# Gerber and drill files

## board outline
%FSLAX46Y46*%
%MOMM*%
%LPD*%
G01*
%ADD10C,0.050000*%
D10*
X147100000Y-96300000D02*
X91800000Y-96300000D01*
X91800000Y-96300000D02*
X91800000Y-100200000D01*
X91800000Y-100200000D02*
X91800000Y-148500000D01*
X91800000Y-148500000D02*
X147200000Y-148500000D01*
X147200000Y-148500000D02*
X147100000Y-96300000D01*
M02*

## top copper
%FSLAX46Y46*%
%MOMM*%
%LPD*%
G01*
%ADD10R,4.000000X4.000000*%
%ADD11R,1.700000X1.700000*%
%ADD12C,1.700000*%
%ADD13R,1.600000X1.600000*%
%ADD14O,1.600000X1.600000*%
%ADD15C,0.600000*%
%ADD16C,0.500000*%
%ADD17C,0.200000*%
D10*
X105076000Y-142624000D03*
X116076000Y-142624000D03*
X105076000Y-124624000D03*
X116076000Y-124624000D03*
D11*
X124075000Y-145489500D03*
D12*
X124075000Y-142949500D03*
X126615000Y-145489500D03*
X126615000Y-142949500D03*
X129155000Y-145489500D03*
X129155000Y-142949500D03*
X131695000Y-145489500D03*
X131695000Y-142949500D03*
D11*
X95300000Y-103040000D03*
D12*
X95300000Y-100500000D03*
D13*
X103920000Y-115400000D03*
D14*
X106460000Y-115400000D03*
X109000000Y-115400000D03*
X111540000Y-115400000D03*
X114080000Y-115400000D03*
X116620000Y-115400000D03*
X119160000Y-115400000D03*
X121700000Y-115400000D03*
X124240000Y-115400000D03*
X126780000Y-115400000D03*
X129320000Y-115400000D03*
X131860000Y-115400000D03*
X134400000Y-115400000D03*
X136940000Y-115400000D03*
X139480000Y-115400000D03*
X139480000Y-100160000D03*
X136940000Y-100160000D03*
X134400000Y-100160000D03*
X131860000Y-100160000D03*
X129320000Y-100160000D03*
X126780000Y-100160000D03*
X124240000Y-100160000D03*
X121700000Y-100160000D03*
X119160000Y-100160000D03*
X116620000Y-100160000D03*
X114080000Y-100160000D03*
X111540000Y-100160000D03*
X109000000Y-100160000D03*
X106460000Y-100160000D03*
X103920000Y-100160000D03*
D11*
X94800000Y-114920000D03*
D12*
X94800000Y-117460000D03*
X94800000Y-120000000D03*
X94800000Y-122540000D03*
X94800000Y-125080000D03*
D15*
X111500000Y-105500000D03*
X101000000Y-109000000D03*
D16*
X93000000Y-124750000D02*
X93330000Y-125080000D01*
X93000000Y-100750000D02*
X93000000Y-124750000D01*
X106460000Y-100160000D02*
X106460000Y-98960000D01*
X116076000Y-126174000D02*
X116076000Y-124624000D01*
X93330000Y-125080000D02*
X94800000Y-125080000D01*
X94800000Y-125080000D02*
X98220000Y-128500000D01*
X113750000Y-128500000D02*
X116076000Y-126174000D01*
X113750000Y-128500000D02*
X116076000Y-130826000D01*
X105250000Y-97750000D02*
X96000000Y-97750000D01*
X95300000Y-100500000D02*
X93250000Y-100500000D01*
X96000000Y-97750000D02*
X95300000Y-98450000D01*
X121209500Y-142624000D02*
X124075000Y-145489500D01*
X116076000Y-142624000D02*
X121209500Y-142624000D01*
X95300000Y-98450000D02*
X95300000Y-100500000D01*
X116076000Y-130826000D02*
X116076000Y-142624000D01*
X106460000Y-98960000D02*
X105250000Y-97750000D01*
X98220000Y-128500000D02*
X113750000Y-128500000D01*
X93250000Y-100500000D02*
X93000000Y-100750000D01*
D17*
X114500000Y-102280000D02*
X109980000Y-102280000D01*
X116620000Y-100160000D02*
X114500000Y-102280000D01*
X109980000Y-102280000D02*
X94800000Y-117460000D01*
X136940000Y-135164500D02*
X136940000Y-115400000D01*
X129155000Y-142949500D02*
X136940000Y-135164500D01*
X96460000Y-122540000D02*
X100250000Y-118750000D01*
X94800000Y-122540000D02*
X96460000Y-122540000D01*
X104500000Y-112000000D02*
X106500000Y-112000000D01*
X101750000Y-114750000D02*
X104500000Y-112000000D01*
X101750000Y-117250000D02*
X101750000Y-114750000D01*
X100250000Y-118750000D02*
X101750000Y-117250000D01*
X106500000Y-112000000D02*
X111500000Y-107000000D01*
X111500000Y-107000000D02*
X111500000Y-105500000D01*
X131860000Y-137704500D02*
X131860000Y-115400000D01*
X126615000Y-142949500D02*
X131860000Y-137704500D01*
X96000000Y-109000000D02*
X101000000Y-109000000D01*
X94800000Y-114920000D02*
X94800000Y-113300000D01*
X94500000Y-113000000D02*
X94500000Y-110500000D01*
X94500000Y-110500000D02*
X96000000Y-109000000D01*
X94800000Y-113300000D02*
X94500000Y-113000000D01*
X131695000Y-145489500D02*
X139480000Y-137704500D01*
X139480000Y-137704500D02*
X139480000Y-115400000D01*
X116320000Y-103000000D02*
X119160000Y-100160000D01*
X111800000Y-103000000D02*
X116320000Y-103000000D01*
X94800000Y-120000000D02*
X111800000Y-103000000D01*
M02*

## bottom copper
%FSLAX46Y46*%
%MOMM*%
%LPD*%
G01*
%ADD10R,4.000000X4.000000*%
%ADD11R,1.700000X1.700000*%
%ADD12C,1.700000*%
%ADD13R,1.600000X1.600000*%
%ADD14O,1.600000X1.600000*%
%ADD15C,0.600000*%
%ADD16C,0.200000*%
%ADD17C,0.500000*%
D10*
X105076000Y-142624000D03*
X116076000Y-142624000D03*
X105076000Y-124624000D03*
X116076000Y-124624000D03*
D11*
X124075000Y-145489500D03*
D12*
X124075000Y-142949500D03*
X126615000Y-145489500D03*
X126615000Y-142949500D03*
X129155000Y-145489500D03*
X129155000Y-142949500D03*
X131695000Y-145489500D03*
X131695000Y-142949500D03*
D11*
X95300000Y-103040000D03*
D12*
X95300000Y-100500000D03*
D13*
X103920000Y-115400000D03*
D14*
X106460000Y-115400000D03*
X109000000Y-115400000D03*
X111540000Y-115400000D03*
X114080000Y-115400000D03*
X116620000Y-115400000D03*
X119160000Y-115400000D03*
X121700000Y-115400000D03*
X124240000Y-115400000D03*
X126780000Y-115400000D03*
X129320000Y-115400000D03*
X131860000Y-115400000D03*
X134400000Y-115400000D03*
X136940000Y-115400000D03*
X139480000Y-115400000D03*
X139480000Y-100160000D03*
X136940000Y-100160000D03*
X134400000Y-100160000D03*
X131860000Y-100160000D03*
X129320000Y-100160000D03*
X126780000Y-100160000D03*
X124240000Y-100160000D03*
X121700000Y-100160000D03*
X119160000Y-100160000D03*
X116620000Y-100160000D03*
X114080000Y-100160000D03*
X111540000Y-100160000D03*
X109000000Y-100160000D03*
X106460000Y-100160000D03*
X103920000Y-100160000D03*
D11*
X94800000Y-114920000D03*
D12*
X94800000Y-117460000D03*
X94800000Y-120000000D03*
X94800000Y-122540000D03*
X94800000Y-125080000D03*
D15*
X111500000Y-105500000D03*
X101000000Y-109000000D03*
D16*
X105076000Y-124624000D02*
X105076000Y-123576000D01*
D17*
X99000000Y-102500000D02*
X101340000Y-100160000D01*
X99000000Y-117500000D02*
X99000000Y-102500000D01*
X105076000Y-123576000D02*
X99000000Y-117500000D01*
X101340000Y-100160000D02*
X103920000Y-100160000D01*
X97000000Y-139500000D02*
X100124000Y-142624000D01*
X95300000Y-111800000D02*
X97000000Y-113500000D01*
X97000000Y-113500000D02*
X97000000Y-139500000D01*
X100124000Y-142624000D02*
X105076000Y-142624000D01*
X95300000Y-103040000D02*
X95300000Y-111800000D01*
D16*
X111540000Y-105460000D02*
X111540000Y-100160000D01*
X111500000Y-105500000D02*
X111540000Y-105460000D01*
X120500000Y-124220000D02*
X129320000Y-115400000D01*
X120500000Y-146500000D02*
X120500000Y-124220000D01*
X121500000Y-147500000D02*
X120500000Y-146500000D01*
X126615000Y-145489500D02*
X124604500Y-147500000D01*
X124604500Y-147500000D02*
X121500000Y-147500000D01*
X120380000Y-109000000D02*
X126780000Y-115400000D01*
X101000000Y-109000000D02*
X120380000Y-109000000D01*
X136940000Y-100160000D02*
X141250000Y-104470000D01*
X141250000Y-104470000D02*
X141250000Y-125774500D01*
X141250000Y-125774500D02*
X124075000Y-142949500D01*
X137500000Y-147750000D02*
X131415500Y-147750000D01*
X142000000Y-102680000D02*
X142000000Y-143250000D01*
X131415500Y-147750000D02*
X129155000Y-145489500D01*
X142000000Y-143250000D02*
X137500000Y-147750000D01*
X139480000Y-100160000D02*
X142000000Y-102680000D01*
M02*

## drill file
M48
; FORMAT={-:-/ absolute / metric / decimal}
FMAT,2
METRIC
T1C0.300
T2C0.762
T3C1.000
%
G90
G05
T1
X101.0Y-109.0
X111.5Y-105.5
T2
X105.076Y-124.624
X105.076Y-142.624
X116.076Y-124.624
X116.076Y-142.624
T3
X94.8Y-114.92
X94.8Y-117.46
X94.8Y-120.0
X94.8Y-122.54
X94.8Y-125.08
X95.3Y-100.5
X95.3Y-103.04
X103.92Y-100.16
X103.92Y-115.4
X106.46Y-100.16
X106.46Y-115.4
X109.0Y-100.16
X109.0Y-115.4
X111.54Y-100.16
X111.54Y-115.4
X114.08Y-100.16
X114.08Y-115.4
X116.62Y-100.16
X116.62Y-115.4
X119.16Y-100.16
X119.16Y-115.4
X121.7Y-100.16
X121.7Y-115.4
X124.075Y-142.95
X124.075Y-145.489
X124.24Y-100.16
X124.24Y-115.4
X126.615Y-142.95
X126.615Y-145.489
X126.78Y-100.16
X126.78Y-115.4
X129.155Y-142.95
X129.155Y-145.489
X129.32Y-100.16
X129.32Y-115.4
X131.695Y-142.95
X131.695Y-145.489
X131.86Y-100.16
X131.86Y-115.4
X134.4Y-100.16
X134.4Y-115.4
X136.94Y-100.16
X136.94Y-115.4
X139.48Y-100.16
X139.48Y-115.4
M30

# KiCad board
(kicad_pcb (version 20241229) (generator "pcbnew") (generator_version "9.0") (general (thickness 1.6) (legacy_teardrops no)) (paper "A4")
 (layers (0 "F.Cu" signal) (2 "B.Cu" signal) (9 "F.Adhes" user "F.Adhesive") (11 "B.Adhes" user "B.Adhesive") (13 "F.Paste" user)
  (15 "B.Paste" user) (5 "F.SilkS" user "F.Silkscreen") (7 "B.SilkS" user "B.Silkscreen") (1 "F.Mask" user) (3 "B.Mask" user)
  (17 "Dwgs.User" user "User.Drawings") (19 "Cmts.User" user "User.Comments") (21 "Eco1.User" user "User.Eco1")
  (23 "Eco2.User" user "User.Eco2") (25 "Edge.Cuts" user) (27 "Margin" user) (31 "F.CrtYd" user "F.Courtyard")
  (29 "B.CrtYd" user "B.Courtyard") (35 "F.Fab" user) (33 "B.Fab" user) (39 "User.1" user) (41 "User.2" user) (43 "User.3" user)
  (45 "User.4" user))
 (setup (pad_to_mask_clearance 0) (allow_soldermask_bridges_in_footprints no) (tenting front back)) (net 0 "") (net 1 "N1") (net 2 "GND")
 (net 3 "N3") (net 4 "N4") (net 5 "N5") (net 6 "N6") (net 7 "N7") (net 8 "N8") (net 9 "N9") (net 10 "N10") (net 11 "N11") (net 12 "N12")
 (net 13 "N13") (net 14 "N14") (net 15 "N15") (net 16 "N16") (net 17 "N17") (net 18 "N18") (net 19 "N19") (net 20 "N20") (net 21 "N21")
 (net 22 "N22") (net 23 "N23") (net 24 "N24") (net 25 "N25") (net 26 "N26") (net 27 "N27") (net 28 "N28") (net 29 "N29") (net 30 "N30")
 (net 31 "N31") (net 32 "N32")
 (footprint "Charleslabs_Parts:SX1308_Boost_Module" (layer "F.Cu") (at 105.124 142.576 90)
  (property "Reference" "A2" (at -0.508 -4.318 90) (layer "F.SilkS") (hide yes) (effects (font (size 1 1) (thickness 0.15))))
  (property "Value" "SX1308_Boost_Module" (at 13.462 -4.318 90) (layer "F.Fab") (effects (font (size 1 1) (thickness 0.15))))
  (pad "1" thru_hole rect (at -0.048 -0.048 90) (size 4 4) (drill 0.762) (layers "*.Cu" "*.Mask") (remove_unused_layers no) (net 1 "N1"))
  (pad "2" thru_hole rect (at -0.048 10.952 90) (size 4 4) (drill 0.762) (layers "*.Cu" "*.Mask") (remove_unused_layers no) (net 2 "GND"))
  (pad "3" thru_hole rect (at 17.952 -0.048 90) (size 4 4) (drill 0.762) (layers "*.Cu" "*.Mask") (remove_unused_layers no) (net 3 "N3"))
  (pad "4" thru_hole rect (at 17.952 10.952 90) (size 4 4) (drill 0.762) (layers "*.Cu" "*.Mask") (remove_unused_layers no) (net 2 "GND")))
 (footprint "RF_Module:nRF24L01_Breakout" (layer "F.Cu") (at 124.075 145.4895 90)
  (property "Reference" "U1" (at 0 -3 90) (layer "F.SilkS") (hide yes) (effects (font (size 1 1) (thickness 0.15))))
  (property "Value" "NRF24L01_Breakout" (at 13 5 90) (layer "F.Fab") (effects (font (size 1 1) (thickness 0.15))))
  (pad "1" thru_hole rect (at 0 0 90) (size 1.7 1.7) (drill 1) (layers "*.Cu" "*.Mask") (remove_unused_layers no) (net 2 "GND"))
  (pad "2" thru_hole circle (at 2.54 0 90) (size 1.7 1.7) (drill 1) (layers "*.Cu" "*.Mask") (remove_unused_layers no) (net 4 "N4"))
  (pad "3" thru_hole circle (at 0 2.54 90) (size 1.7 1.7) (drill 1) (layers "*.Cu" "*.Mask") (remove_unused_layers no) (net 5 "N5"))
  (pad "4" thru_hole circle (at 2.54 2.54 90) (size 1.7 1.7) (drill 1) (layers "*.Cu" "*.Mask") (remove_unused_layers no) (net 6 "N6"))
  (pad "5" thru_hole circle (at 0 5.08 90) (size 1.7 1.7) (drill 1) (layers "*.Cu" "*.Mask") (remove_unused_layers no) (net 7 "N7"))
  (pad "6" thru_hole circle (at 2.54 5.08 90) (size 1.7 1.7) (drill 1) (layers "*.Cu" "*.Mask") (remove_unused_layers no) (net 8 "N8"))
  (pad "7" thru_hole circle (at 0 7.62 90) (size 1.7 1.7) (drill 1) (layers "*.Cu" "*.Mask") (remove_unused_layers no) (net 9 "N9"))
  (pad "8" thru_hole circle (at 2.54 7.62 90) (size 1.7 1.7) (drill 1) (layers "*.Cu" "*.Mask") (remove_unused_layers no) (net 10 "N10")))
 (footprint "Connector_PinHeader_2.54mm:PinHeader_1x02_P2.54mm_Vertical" (layer "F.Cu") (at 95.3 103.04 180)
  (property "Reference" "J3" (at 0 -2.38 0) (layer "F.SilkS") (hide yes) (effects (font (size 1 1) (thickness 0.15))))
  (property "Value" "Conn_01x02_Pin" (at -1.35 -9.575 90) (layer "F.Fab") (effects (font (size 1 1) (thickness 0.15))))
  (pad "1" thru_hole rect (at 0 0 180) (size 1.7 1.7) (drill 1) (layers "*.Cu" "*.Mask") (remove_unused_layers no) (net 1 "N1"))
  (pad "2" thru_hole circle (at 0 2.54 180) (size 1.7 1.7) (drill 1) (layers "*.Cu" "*.Mask") (remove_unused_layers no) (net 2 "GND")))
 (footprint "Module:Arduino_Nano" (layer "F.Cu") (at 103.92 115.4 90)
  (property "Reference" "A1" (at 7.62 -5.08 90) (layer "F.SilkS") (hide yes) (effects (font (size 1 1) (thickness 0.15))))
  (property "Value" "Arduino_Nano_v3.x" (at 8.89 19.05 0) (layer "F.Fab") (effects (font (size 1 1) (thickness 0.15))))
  (pad "1" thru_hole rect (at 0 0 90) (size 1.6 1.6) (drill 1) (layers "*.Cu" "*.Mask") (remove_unused_layers no) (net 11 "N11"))
  (pad "2" thru_hole oval (at 0 2.54 90) (size 1.6 1.6) (drill 1) (layers "*.Cu" "*.Mask") (remove_unused_layers no) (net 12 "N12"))
  (pad "3" thru_hole oval (at 0 5.08 90) (size 1.6 1.6) (drill 1) (layers "*.Cu" "*.Mask") (remove_unused_layers no) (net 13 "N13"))
  (pad "4" thru_hole oval (at 0 7.62 90) (size 1.6 1.6) (drill 1) (layers "*.Cu" "*.Mask") (remove_unused_layers no) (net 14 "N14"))
  (pad "5" thru_hole oval (at 0 10.16 90) (size 1.6 1.6) (drill 1) (layers "*.Cu" "*.Mask") (remove_unused_layers no) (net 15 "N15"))
  (pad "6" thru_hole oval (at 0 12.7 90) (size 1.6 1.6) (drill 1) (layers "*.Cu" "*.Mask") (remove_unused_layers no) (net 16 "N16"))
  (pad "7" thru_hole oval (at 0 15.24 90) (size 1.6 1.6) (drill 1) (layers "*.Cu" "*.Mask") (remove_unused_layers no) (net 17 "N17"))
  (pad "8" thru_hole oval (at 0 17.78 90) (size 1.6 1.6) (drill 1) (layers "*.Cu" "*.Mask") (remove_unused_layers no) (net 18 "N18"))
  (pad "9" thru_hole oval (at 0 20.32 90) (size 1.6 1.6) (drill 1) (layers "*.Cu" "*.Mask") (remove_unused_layers no) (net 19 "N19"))
  (pad "10" thru_hole oval (at 0 22.86 90) (size 1.6 1.6) (drill 1) (layers "*.Cu" "*.Mask") (remove_unused_layers no) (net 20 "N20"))
  (pad "11" thru_hole oval (at 0 25.4 90) (size 1.6 1.6) (drill 1) (layers "*.Cu" "*.Mask") (remove_unused_layers no) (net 5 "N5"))
  (pad "12" thru_hole oval (at 0 27.94 90) (size 1.6 1.6) (drill 1) (layers "*.Cu" "*.Mask") (remove_unused_layers no) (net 6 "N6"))
  (pad "13" thru_hole oval (at 0 30.48 90) (size 1.6 1.6) (drill 1) (layers "*.Cu" "*.Mask") (remove_unused_layers no) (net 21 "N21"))
  (pad "14" thru_hole oval (at 0 33.02 90) (size 1.6 1.6) (drill 1) (layers "*.Cu" "*.Mask") (remove_unused_layers no) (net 8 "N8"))
  (pad "15" thru_hole oval (at 0 35.56 90) (size 1.6 1.6) (drill 1) (layers "*.Cu" "*.Mask") (remove_unused_layers no) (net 9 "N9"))
  (pad "16" thru_hole oval (at 15.24 35.56 90) (size 1.6 1.6) (drill 1) (layers "*.Cu" "*.Mask") (remove_unused_layers no) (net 7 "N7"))
  (pad "17" thru_hole oval (at 15.24 33.02 90) (size 1.6 1.6) (drill 1) (layers "*.Cu" "*.Mask") (remove_unused_layers no) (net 4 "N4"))
  (pad "18" thru_hole oval (at 15.24 30.48 90) (size 1.6 1.6) (drill 1) (layers "*.Cu" "*.Mask") (remove_unused_layers no) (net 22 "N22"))
  (pad "19" thru_hole oval (at 15.24 27.94 90) (size 1.6 1.6) (drill 1) (layers "*.Cu" "*.Mask") (remove_unused_layers no) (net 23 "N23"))
  (pad "20" thru_hole oval (at 15.24 25.4 90) (size 1.6 1.6) (drill 1) (layers "*.Cu" "*.Mask") (remove_unused_layers no) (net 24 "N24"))
  (pad "21" thru_hole oval (at 15.24 22.86 90) (size 1.6 1.6) (drill 1) (layers "*.Cu" "*.Mask") (remove_unused_layers no) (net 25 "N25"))
  (pad "22" thru_hole oval (at 15.24 20.32 90) (size 1.6 1.6) (drill 1) (layers "*.Cu" "*.Mask") (remove_unused_layers no) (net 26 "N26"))
  (pad "23" thru_hole oval (at 15.24 17.78 90) (size 1.6 1.6) (drill 1) (layers "*.Cu" "*.Mask") (remove_unused_layers no) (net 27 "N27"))
  (pad "24" thru_hole oval (at 15.24 15.24 90) (size 1.6 1.6) (drill 1) (layers "*.Cu" "*.Mask") (remove_unused_layers no) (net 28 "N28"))
  (pad "25" thru_hole oval (at 15.24 12.7 90) (size 1.6 1.6) (drill 1) (layers "*.Cu" "*.Mask") (remove_unused_layers no) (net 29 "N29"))
  (pad "26" thru_hole oval (at 15.24 10.16 90) (size 1.6 1.6) (drill 1) (layers "*.Cu" "*.Mask") (remove_unused_layers no) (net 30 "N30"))
  (pad "27" thru_hole oval (at 15.24 7.62 90) (size 1.6 1.6) (drill 1) (layers "*.Cu" "*.Mask") (remove_unused_layers no) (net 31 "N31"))
  (pad "28" thru_hole oval (at 15.24 5.08 90) (size 1.6 1.6) (drill 1) (layers "*.Cu" "*.Mask") (remove_unused_layers no) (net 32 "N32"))
  (pad "29" thru_hole oval (at 15.24 2.54 90) (size 1.6 1.6) (drill 1) (layers "*.Cu" "*.Mask") (remove_unused_layers no) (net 2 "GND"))
  (pad "30" thru_hole oval (at 15.24 0 90) (size 1.6 1.6) (drill 1) (layers "*.Cu" "*.Mask") (remove_unused_layers no) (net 3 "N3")))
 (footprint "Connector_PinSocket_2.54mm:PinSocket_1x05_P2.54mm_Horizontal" (layer "F.Cu") (at 94.8 114.92)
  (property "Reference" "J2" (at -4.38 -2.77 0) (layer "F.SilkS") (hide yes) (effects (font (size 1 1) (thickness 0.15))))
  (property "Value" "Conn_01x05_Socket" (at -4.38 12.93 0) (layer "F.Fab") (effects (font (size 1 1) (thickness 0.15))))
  (pad "1" thru_hole rect (at 0 0) (size 1.7 1.7) (drill 1) (layers "*.Cu" "*.Mask") (remove_unused_layers no) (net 20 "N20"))
  (pad "2" thru_hole circle (at 0 2.54) (size 1.7 1.7) (drill 1) (layers "*.Cu" "*.Mask") (remove_unused_layers no) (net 29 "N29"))
  (pad "3" thru_hole circle (at 0 5.08) (size 1.7 1.7) (drill 1) (layers "*.Cu" "*.Mask") (remove_unused_layers no) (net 28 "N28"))
  (pad "4" thru_hole circle (at 0 7.62) (size 1.7 1.7) (drill 1) (layers "*.Cu" "*.Mask") (remove_unused_layers no) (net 31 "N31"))
  (pad "5" thru_hole circle (at 0 10.16) (size 1.7 1.7) (drill 1) (layers "*.Cu" "*.Mask") (remove_unused_layers no) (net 2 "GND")))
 (gr_line (start 147.1 96.3) (end 91.8 96.3) (stroke (width 0.05) (type default)) (layer "Edge.Cuts"))
 (gr_line (start 91.8 96.3) (end 91.8 100.2) (stroke (width 0.05) (type default)) (layer "Edge.Cuts"))
 (gr_line (start 91.8 100.2) (end 91.8 148.5) (stroke (width 0.05) (type default)) (layer "Edge.Cuts"))
 (gr_line (start 91.8 148.5) (end 147.2 148.5) (stroke (width 0.05) (type default)) (layer "Edge.Cuts"))
 (gr_line (start 147.2 148.5) (end 147.1 96.3) (stroke (width 0.05) (type default)) (layer "Edge.Cuts"))
 (segment (start 93 124.75) (end 93.33 125.08) (width 0.5) (layer "F.Cu") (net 2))
 (segment (start 93 100.75) (end 93 124.75) (width 0.5) (layer "F.Cu") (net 2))
 (segment (start 106.46 100.16) (end 106.46 98.96) (width 0.5) (layer "F.Cu") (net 2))
 (segment (start 116.076 126.174) (end 116.076 124.624) (width 0.5) (layer "F.Cu") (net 2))
 (segment (start 93.33 125.08) (end 94.8 125.08) (width 0.5) (layer "F.Cu") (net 2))
 (segment (start 94.8 125.08) (end 98.22 128.5) (width 0.5) (layer "F.Cu") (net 2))
 (segment (start 113.75 128.5) (end 116.076 126.174) (width 0.5) (layer "F.Cu") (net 2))
 (segment (start 113.75 128.5) (end 116.076 130.826) (width 0.5) (layer "F.Cu") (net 2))
 (segment (start 105.25 97.75) (end 96 97.75) (width 0.5) (layer "F.Cu") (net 2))
 (segment (start 95.3 100.5) (end 93.25 100.5) (width 0.5) (layer "F.Cu") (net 2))
 (segment (start 96 97.75) (end 95.3 98.45) (width 0.5) (layer "F.Cu") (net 2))
 (segment (start 121.2095 142.624) (end 124.075 145.4895) (width 0.5) (layer "F.Cu") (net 2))
 (segment (start 116.076 142.624) (end 121.2095 142.624) (width 0.5) (layer "F.Cu") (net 2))
 (segment (start 95.3 98.45) (end 95.3 100.5) (width 0.5) (layer "F.Cu") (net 2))
 (segment (start 116.076 130.826) (end 116.076 142.624) (width 0.5) (layer "F.Cu") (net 2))
 (segment (start 106.46 98.96) (end 105.25 97.75) (width 0.5) (layer "F.Cu") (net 2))
 (segment (start 98.22 128.5) (end 113.75 128.5) (width 0.5) (layer "F.Cu") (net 2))
 (segment (start 93.25 100.5) (end 93 100.75) (width 0.5) (layer "F.Cu") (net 2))
 (segment (start 105.076 124.624) (end 105.076 123.576) (width 0.2) (layer "B.Cu") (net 3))
 (segment (start 99 102.5) (end 101.34 100.16) (width 0.5) (layer "B.Cu") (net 3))
 (segment (start 99 117.5) (end 99 102.5) (width 0.5) (layer "B.Cu") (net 3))
 (segment (start 105.076 123.576) (end 99 117.5) (width 0.5) (layer "B.Cu") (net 3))
 (segment (start 101.34 100.16) (end 103.92 100.16) (width 0.5) (layer "B.Cu") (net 3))
 (segment (start 97 139.5) (end 100.124 142.624) (width 0.5) (layer "B.Cu") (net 1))
 (segment (start 95.3 111.8) (end 97 113.5) (width 0.5) (layer "B.Cu") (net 1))
 (segment (start 97 113.5) (end 97 139.5) (width 0.5) (layer "B.Cu") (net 1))
 (segment (start 100.124 142.624) (end 105.076 142.624) (width 0.5) (layer "B.Cu") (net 1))
 (segment (start 95.3 103.04) (end 95.3 111.8) (width 0.5) (layer "B.Cu") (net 1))
 (segment (start 114.5 102.28) (end 109.98 102.28) (width 0.2) (layer "F.Cu") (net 29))
 (segment (start 116.62 100.16) (end 114.5 102.28) (width 0.2) (layer "F.Cu") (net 29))
 (segment (start 109.98 102.28) (end 94.8 117.46) (width 0.2) (layer "F.Cu") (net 29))
 (segment (start 136.94 135.1645) (end 136.94 115.4) (width 0.2) (layer "F.Cu") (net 8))
 (segment (start 129.155 142.9495) (end 136.94 135.1645) (width 0.2) (layer "F.Cu") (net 8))
 (segment (start 96.46 122.54) (end 100.25 118.75) (width 0.2) (layer "F.Cu") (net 31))
 (segment (start 94.8 122.54) (end 96.46 122.54) (width 0.2) (layer "F.Cu") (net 31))
 (segment (start 104.5 112) (end 106.5 112) (width 0.2) (layer "F.Cu") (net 31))
 (segment (start 101.75 114.75) (end 104.5 112) (width 0.2) (layer "F.Cu") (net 31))
 (segment (start 101.75 117.25) (end 101.75 114.75) (width 0.2) (layer "F.Cu") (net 31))
 (segment (start 100.25 118.75) (end 101.75 117.25) (width 0.2) (layer "F.Cu") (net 31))
 (segment (start 106.5 112) (end 111.5 107) (width 0.2) (layer "F.Cu") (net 31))
 (segment (start 111.5 107) (end 111.5 105.5) (width 0.2) (layer "F.Cu") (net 31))
 (via (at 111.5 105.5) (size 0.6) (drill 0.3) (layers "F.Cu" "B.Cu") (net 31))
 (segment (start 111.54 105.46) (end 111.54 100.16) (width 0.2) (layer "B.Cu") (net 31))
 (segment (start 111.5 105.5) (end 111.54 105.46) (width 0.2) (layer "B.Cu") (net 31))
 (segment (start 131.86 137.7045) (end 131.86 115.4) (width 0.2) (layer "F.Cu") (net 6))
 (segment (start 126.615 142.9495) (end 131.86 137.7045) (width 0.2) (layer "F.Cu") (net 6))
 (segment (start 120.5 124.22) (end 129.32 115.4) (width 0.2) (layer "B.Cu") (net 5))
 (segment (start 120.5 146.5) (end 120.5 124.22) (width 0.2) (layer "B.Cu") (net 5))
 (segment (start 121.5 147.5) (end 120.5 146.5) (width 0.2) (layer "B.Cu") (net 5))
 (segment (start 126.615 145.4895) (end 124.6045 147.5) (width 0.2) (layer "B.Cu") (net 5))
 (segment (start 124.6045 147.5) (end 121.5 147.5) (width 0.2) (layer "B.Cu") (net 5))
 (segment (start 96 109) (end 101 109) (width 0.2) (layer "F.Cu") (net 20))
 (segment (start 94.8 114.92) (end 94.8 113.3) (width 0.2) (layer "F.Cu") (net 20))
 (segment (start 94.5 113) (end 94.5 110.5) (width 0.2) (layer "F.Cu") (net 20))
 (segment (start 94.5 110.5) (end 96 109) (width 0.2) (layer "F.Cu") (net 20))
 (segment (start 94.8 113.3) (end 94.5 113) (width 0.2) (layer "F.Cu") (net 20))
 (via (at 101 109) (size 0.6) (drill 0.3) (layers "F.Cu" "B.Cu") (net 20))
 (segment (start 120.38 109) (end 126.78 115.4) (width 0.2) (layer "B.Cu") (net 20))
 (segment (start 101 109) (end 120.38 109) (width 0.2) (layer "B.Cu") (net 20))
 (segment (start 131.695 145.4895) (end 139.48 137.7045) (width 0.2) (layer "F.Cu") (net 9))
 (segment (start 139.48 137.7045) (end 139.48 115.4) (width 0.2) (layer "F.Cu") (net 9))
 (segment (start 136.94 100.16) (end 141.25 104.47) (width 0.2) (layer "B.Cu") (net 4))
 (segment (start 141.25 104.47) (end 141.25 125.7745) (width 0.2) (layer "B.Cu") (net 4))
 (segment (start 141.25 125.7745) (end 124.075 142.9495) (width 0.2) (layer "B.Cu") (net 4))
 (segment (start 116.32 103) (end 119.16 100.16) (width 0.2) (layer "F.Cu") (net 28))
 (segment (start 111.8 103) (end 116.32 103) (width 0.2) (layer "F.Cu") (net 28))
 (segment (start 94.8 120) (end 111.8 103) (width 0.2) (layer "F.Cu") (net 28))
 (segment (start 137.5 147.75) (end 131.4155 147.75) (width 0.2) (layer "B.Cu") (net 7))
 (segment (start 142 102.68) (end 142 143.25) (width 0.2) (layer "B.Cu") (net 7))
 (segment (start 131.4155 147.75) (end 129.155 145.4895) (width 0.2) (layer "B.Cu") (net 7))
 (segment (start 142 143.25) (end 137.5 147.75) (width 0.2) (layer "B.Cu") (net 7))
 (segment (start 139.48 100.16) (end 142 102.68) (width 0.2) (layer "B.Cu") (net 7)))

